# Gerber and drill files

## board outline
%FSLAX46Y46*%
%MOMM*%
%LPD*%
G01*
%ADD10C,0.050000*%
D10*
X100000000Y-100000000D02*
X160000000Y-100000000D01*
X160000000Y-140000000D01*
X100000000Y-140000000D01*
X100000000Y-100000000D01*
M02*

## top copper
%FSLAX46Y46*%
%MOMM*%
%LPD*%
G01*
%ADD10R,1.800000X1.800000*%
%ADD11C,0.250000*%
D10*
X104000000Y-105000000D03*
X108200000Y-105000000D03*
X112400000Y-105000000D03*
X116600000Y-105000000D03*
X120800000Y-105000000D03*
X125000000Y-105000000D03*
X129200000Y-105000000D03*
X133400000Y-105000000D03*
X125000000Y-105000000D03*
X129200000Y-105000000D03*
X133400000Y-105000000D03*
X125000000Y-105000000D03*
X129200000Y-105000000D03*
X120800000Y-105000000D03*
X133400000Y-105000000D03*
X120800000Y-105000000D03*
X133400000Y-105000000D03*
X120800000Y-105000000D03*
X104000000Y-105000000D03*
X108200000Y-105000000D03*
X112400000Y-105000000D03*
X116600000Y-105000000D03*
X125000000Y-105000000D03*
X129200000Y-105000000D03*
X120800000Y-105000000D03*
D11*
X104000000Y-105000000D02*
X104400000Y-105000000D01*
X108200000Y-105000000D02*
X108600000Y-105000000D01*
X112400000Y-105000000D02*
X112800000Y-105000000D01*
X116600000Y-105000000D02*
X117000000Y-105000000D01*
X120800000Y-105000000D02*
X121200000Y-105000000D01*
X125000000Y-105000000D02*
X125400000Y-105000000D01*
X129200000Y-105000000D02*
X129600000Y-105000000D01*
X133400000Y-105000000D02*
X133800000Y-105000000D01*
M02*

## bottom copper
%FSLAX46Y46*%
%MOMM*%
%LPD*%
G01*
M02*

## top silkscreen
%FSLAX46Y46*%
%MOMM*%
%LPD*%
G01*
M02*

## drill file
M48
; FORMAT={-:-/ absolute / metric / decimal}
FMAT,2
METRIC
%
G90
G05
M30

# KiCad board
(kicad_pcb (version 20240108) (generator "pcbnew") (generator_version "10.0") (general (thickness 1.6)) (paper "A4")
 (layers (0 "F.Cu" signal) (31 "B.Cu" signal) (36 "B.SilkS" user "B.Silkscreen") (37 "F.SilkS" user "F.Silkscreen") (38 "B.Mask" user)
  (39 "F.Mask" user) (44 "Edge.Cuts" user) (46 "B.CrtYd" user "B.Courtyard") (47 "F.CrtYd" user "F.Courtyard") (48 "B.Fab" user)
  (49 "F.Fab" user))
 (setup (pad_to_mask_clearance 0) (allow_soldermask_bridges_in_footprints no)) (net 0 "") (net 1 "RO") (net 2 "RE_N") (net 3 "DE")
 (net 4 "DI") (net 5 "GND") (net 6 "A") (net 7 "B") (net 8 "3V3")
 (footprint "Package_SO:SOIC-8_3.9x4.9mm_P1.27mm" (layer "F.Cu") (at 100 100)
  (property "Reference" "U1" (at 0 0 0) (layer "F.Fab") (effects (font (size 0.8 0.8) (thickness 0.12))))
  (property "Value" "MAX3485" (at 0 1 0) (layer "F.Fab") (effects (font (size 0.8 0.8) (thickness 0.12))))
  (pad "1" smd rect (at 4.000 5.000) (size 1.8 1.8) (layers "F.Cu" "F.Paste" "F.Mask") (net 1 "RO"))
  (pad "2" smd rect (at 8.200 5.000) (size 1.8 1.8) (layers "F.Cu" "F.Paste" "F.Mask") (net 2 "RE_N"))
  (pad "3" smd rect (at 12.400 5.000) (size 1.8 1.8) (layers "F.Cu" "F.Paste" "F.Mask") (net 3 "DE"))
  (pad "4" smd rect (at 16.600 5.000) (size 1.8 1.8) (layers "F.Cu" "F.Paste" "F.Mask") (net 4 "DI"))
  (pad "5" smd rect (at 20.800 5.000) (size 1.8 1.8) (layers "F.Cu" "F.Paste" "F.Mask") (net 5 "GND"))
  (pad "6" smd rect (at 25.000 5.000) (size 1.8 1.8) (layers "F.Cu" "F.Paste" "F.Mask") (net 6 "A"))
  (pad "7" smd rect (at 29.200 5.000) (size 1.8 1.8) (layers "F.Cu" "F.Paste" "F.Mask") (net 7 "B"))
  (pad "8" smd rect (at 33.400 5.000) (size 1.8 1.8) (layers "F.Cu" "F.Paste" "F.Mask") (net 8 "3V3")))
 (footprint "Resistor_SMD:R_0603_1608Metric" (layer "F.Cu") (at 100 100)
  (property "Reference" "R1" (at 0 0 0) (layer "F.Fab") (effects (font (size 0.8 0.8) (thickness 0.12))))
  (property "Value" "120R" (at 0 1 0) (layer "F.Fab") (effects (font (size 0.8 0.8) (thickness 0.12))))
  (pad "1" smd rect (at 25.000 5.000) (size 1.8 1.8) (layers "F.Cu" "F.Paste" "F.Mask") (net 6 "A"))
  (pad "2" smd rect (at 29.200 5.000) (size 1.8 1.8) (layers "F.Cu" "F.Paste" "F.Mask") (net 7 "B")))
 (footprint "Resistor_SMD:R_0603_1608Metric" (layer "F.Cu") (at 100 100)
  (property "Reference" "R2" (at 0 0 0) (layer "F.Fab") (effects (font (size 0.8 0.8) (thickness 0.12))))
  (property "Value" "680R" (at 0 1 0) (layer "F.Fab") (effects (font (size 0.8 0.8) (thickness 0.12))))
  (pad "1" smd rect (at 33.400 5.000) (size 1.8 1.8) (layers "F.Cu" "F.Paste" "F.Mask") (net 8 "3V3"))
  (pad "2" smd rect (at 25.000 5.000) (size 1.8 1.8) (layers "F.Cu" "F.Paste" "F.Mask") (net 6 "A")))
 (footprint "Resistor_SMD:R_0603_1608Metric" (layer "F.Cu") (at 100 100)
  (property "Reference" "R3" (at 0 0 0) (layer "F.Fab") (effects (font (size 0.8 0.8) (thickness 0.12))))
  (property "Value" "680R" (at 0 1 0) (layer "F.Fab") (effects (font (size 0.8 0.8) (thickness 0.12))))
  (pad "1" smd rect (at 29.200 5.000) (size 1.8 1.8) (layers "F.Cu" "F.Paste" "F.Mask") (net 7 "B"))
  (pad "2" smd rect (at 20.800 5.000) (size 1.8 1.8) (layers "F.Cu" "F.Paste" "F.Mask") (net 5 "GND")))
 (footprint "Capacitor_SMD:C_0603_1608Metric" (layer "F.Cu") (at 100 100)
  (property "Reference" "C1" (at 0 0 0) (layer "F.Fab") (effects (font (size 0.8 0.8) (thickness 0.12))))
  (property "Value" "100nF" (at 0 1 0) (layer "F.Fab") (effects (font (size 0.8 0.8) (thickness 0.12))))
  (pad "1" smd rect (at 33.400 5.000) (size 1.8 1.8) (layers "F.Cu" "F.Paste" "F.Mask") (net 8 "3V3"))
  (pad "2" smd rect (at 20.800 5.000) (size 1.8 1.8) (layers "F.Cu" "F.Paste" "F.Mask") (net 5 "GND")))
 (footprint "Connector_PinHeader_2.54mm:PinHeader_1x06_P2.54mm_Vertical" (layer "F.Cu") (at 100 100)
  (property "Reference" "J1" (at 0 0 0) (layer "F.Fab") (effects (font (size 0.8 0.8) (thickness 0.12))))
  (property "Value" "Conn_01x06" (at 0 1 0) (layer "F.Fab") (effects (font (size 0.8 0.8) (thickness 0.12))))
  (pad "1" smd rect (at 33.400 5.000) (size 1.8 1.8) (layers "F.Cu" "F.Paste" "F.Mask") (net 8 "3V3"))
  (pad "2" smd rect (at 20.800 5.000) (size 1.8 1.8) (layers "F.Cu" "F.Paste" "F.Mask") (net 5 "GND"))
  (pad "3" smd rect (at 4.000 5.000) (size 1.8 1.8) (layers "F.Cu" "F.Paste" "F.Mask") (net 1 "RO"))
  (pad "4" smd rect (at 8.200 5.000) (size 1.8 1.8) (layers "F.Cu" "F.Paste" "F.Mask") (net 2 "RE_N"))
  (pad "5" smd rect (at 12.400 5.000) (size 1.8 1.8) (layers "F.Cu" "F.Paste" "F.Mask") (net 3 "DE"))
  (pad "6" smd rect (at 16.600 5.000) (size 1.8 1.8) (layers "F.Cu" "F.Paste" "F.Mask") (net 4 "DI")))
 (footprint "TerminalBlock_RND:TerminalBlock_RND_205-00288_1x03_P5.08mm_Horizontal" (layer "F.Cu") (at 100 100)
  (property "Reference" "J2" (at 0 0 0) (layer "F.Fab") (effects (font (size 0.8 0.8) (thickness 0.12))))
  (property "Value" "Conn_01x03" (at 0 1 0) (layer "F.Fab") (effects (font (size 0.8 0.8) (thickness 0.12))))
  (pad "1" smd rect (at 25.000 5.000) (size 1.8 1.8) (layers "F.Cu" "F.Paste" "F.Mask") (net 6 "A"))
  (pad "2" smd rect (at 29.200 5.000) (size 1.8 1.8) (layers "F.Cu" "F.Paste" "F.Mask") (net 7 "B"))
  (pad "3" smd rect (at 20.800 5.000) (size 1.8 1.8) (layers "F.Cu" "F.Paste" "F.Mask") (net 5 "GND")))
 (gr_rect (start 100 100) (end 160 140) (stroke (width 0.05) (type default)) (fill none) (layer "Edge.Cuts"))
 (segment (start 104.000 105.000) (end 104.400 105.000) (width 0.25) (layer "F.Cu") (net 1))
 (segment (start 108.200 105.000) (end 108.600 105.000) (width 0.25) (layer "F.Cu") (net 2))
 (segment (start 112.400 105.000) (end 112.800 105.000) (width 0.25) (layer "F.Cu") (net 3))
 (segment (start 116.600 105.000) (end 117.000 105.000) (width 0.25) (layer "F.Cu") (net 4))
 (segment (start 120.800 105.000) (end 121.200 105.000) (width 0.25) (layer "F.Cu") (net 5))
 (segment (start 125.000 105.000) (end 125.400 105.000) (width 0.25) (layer "F.Cu") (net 6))
 (segment (start 129.200 105.000) (end 129.600 105.000) (width 0.25) (layer "F.Cu") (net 7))
 (segment (start 133.400 105.000) (end 133.800 105.000) (width 0.25) (layer "F.Cu") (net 8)))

